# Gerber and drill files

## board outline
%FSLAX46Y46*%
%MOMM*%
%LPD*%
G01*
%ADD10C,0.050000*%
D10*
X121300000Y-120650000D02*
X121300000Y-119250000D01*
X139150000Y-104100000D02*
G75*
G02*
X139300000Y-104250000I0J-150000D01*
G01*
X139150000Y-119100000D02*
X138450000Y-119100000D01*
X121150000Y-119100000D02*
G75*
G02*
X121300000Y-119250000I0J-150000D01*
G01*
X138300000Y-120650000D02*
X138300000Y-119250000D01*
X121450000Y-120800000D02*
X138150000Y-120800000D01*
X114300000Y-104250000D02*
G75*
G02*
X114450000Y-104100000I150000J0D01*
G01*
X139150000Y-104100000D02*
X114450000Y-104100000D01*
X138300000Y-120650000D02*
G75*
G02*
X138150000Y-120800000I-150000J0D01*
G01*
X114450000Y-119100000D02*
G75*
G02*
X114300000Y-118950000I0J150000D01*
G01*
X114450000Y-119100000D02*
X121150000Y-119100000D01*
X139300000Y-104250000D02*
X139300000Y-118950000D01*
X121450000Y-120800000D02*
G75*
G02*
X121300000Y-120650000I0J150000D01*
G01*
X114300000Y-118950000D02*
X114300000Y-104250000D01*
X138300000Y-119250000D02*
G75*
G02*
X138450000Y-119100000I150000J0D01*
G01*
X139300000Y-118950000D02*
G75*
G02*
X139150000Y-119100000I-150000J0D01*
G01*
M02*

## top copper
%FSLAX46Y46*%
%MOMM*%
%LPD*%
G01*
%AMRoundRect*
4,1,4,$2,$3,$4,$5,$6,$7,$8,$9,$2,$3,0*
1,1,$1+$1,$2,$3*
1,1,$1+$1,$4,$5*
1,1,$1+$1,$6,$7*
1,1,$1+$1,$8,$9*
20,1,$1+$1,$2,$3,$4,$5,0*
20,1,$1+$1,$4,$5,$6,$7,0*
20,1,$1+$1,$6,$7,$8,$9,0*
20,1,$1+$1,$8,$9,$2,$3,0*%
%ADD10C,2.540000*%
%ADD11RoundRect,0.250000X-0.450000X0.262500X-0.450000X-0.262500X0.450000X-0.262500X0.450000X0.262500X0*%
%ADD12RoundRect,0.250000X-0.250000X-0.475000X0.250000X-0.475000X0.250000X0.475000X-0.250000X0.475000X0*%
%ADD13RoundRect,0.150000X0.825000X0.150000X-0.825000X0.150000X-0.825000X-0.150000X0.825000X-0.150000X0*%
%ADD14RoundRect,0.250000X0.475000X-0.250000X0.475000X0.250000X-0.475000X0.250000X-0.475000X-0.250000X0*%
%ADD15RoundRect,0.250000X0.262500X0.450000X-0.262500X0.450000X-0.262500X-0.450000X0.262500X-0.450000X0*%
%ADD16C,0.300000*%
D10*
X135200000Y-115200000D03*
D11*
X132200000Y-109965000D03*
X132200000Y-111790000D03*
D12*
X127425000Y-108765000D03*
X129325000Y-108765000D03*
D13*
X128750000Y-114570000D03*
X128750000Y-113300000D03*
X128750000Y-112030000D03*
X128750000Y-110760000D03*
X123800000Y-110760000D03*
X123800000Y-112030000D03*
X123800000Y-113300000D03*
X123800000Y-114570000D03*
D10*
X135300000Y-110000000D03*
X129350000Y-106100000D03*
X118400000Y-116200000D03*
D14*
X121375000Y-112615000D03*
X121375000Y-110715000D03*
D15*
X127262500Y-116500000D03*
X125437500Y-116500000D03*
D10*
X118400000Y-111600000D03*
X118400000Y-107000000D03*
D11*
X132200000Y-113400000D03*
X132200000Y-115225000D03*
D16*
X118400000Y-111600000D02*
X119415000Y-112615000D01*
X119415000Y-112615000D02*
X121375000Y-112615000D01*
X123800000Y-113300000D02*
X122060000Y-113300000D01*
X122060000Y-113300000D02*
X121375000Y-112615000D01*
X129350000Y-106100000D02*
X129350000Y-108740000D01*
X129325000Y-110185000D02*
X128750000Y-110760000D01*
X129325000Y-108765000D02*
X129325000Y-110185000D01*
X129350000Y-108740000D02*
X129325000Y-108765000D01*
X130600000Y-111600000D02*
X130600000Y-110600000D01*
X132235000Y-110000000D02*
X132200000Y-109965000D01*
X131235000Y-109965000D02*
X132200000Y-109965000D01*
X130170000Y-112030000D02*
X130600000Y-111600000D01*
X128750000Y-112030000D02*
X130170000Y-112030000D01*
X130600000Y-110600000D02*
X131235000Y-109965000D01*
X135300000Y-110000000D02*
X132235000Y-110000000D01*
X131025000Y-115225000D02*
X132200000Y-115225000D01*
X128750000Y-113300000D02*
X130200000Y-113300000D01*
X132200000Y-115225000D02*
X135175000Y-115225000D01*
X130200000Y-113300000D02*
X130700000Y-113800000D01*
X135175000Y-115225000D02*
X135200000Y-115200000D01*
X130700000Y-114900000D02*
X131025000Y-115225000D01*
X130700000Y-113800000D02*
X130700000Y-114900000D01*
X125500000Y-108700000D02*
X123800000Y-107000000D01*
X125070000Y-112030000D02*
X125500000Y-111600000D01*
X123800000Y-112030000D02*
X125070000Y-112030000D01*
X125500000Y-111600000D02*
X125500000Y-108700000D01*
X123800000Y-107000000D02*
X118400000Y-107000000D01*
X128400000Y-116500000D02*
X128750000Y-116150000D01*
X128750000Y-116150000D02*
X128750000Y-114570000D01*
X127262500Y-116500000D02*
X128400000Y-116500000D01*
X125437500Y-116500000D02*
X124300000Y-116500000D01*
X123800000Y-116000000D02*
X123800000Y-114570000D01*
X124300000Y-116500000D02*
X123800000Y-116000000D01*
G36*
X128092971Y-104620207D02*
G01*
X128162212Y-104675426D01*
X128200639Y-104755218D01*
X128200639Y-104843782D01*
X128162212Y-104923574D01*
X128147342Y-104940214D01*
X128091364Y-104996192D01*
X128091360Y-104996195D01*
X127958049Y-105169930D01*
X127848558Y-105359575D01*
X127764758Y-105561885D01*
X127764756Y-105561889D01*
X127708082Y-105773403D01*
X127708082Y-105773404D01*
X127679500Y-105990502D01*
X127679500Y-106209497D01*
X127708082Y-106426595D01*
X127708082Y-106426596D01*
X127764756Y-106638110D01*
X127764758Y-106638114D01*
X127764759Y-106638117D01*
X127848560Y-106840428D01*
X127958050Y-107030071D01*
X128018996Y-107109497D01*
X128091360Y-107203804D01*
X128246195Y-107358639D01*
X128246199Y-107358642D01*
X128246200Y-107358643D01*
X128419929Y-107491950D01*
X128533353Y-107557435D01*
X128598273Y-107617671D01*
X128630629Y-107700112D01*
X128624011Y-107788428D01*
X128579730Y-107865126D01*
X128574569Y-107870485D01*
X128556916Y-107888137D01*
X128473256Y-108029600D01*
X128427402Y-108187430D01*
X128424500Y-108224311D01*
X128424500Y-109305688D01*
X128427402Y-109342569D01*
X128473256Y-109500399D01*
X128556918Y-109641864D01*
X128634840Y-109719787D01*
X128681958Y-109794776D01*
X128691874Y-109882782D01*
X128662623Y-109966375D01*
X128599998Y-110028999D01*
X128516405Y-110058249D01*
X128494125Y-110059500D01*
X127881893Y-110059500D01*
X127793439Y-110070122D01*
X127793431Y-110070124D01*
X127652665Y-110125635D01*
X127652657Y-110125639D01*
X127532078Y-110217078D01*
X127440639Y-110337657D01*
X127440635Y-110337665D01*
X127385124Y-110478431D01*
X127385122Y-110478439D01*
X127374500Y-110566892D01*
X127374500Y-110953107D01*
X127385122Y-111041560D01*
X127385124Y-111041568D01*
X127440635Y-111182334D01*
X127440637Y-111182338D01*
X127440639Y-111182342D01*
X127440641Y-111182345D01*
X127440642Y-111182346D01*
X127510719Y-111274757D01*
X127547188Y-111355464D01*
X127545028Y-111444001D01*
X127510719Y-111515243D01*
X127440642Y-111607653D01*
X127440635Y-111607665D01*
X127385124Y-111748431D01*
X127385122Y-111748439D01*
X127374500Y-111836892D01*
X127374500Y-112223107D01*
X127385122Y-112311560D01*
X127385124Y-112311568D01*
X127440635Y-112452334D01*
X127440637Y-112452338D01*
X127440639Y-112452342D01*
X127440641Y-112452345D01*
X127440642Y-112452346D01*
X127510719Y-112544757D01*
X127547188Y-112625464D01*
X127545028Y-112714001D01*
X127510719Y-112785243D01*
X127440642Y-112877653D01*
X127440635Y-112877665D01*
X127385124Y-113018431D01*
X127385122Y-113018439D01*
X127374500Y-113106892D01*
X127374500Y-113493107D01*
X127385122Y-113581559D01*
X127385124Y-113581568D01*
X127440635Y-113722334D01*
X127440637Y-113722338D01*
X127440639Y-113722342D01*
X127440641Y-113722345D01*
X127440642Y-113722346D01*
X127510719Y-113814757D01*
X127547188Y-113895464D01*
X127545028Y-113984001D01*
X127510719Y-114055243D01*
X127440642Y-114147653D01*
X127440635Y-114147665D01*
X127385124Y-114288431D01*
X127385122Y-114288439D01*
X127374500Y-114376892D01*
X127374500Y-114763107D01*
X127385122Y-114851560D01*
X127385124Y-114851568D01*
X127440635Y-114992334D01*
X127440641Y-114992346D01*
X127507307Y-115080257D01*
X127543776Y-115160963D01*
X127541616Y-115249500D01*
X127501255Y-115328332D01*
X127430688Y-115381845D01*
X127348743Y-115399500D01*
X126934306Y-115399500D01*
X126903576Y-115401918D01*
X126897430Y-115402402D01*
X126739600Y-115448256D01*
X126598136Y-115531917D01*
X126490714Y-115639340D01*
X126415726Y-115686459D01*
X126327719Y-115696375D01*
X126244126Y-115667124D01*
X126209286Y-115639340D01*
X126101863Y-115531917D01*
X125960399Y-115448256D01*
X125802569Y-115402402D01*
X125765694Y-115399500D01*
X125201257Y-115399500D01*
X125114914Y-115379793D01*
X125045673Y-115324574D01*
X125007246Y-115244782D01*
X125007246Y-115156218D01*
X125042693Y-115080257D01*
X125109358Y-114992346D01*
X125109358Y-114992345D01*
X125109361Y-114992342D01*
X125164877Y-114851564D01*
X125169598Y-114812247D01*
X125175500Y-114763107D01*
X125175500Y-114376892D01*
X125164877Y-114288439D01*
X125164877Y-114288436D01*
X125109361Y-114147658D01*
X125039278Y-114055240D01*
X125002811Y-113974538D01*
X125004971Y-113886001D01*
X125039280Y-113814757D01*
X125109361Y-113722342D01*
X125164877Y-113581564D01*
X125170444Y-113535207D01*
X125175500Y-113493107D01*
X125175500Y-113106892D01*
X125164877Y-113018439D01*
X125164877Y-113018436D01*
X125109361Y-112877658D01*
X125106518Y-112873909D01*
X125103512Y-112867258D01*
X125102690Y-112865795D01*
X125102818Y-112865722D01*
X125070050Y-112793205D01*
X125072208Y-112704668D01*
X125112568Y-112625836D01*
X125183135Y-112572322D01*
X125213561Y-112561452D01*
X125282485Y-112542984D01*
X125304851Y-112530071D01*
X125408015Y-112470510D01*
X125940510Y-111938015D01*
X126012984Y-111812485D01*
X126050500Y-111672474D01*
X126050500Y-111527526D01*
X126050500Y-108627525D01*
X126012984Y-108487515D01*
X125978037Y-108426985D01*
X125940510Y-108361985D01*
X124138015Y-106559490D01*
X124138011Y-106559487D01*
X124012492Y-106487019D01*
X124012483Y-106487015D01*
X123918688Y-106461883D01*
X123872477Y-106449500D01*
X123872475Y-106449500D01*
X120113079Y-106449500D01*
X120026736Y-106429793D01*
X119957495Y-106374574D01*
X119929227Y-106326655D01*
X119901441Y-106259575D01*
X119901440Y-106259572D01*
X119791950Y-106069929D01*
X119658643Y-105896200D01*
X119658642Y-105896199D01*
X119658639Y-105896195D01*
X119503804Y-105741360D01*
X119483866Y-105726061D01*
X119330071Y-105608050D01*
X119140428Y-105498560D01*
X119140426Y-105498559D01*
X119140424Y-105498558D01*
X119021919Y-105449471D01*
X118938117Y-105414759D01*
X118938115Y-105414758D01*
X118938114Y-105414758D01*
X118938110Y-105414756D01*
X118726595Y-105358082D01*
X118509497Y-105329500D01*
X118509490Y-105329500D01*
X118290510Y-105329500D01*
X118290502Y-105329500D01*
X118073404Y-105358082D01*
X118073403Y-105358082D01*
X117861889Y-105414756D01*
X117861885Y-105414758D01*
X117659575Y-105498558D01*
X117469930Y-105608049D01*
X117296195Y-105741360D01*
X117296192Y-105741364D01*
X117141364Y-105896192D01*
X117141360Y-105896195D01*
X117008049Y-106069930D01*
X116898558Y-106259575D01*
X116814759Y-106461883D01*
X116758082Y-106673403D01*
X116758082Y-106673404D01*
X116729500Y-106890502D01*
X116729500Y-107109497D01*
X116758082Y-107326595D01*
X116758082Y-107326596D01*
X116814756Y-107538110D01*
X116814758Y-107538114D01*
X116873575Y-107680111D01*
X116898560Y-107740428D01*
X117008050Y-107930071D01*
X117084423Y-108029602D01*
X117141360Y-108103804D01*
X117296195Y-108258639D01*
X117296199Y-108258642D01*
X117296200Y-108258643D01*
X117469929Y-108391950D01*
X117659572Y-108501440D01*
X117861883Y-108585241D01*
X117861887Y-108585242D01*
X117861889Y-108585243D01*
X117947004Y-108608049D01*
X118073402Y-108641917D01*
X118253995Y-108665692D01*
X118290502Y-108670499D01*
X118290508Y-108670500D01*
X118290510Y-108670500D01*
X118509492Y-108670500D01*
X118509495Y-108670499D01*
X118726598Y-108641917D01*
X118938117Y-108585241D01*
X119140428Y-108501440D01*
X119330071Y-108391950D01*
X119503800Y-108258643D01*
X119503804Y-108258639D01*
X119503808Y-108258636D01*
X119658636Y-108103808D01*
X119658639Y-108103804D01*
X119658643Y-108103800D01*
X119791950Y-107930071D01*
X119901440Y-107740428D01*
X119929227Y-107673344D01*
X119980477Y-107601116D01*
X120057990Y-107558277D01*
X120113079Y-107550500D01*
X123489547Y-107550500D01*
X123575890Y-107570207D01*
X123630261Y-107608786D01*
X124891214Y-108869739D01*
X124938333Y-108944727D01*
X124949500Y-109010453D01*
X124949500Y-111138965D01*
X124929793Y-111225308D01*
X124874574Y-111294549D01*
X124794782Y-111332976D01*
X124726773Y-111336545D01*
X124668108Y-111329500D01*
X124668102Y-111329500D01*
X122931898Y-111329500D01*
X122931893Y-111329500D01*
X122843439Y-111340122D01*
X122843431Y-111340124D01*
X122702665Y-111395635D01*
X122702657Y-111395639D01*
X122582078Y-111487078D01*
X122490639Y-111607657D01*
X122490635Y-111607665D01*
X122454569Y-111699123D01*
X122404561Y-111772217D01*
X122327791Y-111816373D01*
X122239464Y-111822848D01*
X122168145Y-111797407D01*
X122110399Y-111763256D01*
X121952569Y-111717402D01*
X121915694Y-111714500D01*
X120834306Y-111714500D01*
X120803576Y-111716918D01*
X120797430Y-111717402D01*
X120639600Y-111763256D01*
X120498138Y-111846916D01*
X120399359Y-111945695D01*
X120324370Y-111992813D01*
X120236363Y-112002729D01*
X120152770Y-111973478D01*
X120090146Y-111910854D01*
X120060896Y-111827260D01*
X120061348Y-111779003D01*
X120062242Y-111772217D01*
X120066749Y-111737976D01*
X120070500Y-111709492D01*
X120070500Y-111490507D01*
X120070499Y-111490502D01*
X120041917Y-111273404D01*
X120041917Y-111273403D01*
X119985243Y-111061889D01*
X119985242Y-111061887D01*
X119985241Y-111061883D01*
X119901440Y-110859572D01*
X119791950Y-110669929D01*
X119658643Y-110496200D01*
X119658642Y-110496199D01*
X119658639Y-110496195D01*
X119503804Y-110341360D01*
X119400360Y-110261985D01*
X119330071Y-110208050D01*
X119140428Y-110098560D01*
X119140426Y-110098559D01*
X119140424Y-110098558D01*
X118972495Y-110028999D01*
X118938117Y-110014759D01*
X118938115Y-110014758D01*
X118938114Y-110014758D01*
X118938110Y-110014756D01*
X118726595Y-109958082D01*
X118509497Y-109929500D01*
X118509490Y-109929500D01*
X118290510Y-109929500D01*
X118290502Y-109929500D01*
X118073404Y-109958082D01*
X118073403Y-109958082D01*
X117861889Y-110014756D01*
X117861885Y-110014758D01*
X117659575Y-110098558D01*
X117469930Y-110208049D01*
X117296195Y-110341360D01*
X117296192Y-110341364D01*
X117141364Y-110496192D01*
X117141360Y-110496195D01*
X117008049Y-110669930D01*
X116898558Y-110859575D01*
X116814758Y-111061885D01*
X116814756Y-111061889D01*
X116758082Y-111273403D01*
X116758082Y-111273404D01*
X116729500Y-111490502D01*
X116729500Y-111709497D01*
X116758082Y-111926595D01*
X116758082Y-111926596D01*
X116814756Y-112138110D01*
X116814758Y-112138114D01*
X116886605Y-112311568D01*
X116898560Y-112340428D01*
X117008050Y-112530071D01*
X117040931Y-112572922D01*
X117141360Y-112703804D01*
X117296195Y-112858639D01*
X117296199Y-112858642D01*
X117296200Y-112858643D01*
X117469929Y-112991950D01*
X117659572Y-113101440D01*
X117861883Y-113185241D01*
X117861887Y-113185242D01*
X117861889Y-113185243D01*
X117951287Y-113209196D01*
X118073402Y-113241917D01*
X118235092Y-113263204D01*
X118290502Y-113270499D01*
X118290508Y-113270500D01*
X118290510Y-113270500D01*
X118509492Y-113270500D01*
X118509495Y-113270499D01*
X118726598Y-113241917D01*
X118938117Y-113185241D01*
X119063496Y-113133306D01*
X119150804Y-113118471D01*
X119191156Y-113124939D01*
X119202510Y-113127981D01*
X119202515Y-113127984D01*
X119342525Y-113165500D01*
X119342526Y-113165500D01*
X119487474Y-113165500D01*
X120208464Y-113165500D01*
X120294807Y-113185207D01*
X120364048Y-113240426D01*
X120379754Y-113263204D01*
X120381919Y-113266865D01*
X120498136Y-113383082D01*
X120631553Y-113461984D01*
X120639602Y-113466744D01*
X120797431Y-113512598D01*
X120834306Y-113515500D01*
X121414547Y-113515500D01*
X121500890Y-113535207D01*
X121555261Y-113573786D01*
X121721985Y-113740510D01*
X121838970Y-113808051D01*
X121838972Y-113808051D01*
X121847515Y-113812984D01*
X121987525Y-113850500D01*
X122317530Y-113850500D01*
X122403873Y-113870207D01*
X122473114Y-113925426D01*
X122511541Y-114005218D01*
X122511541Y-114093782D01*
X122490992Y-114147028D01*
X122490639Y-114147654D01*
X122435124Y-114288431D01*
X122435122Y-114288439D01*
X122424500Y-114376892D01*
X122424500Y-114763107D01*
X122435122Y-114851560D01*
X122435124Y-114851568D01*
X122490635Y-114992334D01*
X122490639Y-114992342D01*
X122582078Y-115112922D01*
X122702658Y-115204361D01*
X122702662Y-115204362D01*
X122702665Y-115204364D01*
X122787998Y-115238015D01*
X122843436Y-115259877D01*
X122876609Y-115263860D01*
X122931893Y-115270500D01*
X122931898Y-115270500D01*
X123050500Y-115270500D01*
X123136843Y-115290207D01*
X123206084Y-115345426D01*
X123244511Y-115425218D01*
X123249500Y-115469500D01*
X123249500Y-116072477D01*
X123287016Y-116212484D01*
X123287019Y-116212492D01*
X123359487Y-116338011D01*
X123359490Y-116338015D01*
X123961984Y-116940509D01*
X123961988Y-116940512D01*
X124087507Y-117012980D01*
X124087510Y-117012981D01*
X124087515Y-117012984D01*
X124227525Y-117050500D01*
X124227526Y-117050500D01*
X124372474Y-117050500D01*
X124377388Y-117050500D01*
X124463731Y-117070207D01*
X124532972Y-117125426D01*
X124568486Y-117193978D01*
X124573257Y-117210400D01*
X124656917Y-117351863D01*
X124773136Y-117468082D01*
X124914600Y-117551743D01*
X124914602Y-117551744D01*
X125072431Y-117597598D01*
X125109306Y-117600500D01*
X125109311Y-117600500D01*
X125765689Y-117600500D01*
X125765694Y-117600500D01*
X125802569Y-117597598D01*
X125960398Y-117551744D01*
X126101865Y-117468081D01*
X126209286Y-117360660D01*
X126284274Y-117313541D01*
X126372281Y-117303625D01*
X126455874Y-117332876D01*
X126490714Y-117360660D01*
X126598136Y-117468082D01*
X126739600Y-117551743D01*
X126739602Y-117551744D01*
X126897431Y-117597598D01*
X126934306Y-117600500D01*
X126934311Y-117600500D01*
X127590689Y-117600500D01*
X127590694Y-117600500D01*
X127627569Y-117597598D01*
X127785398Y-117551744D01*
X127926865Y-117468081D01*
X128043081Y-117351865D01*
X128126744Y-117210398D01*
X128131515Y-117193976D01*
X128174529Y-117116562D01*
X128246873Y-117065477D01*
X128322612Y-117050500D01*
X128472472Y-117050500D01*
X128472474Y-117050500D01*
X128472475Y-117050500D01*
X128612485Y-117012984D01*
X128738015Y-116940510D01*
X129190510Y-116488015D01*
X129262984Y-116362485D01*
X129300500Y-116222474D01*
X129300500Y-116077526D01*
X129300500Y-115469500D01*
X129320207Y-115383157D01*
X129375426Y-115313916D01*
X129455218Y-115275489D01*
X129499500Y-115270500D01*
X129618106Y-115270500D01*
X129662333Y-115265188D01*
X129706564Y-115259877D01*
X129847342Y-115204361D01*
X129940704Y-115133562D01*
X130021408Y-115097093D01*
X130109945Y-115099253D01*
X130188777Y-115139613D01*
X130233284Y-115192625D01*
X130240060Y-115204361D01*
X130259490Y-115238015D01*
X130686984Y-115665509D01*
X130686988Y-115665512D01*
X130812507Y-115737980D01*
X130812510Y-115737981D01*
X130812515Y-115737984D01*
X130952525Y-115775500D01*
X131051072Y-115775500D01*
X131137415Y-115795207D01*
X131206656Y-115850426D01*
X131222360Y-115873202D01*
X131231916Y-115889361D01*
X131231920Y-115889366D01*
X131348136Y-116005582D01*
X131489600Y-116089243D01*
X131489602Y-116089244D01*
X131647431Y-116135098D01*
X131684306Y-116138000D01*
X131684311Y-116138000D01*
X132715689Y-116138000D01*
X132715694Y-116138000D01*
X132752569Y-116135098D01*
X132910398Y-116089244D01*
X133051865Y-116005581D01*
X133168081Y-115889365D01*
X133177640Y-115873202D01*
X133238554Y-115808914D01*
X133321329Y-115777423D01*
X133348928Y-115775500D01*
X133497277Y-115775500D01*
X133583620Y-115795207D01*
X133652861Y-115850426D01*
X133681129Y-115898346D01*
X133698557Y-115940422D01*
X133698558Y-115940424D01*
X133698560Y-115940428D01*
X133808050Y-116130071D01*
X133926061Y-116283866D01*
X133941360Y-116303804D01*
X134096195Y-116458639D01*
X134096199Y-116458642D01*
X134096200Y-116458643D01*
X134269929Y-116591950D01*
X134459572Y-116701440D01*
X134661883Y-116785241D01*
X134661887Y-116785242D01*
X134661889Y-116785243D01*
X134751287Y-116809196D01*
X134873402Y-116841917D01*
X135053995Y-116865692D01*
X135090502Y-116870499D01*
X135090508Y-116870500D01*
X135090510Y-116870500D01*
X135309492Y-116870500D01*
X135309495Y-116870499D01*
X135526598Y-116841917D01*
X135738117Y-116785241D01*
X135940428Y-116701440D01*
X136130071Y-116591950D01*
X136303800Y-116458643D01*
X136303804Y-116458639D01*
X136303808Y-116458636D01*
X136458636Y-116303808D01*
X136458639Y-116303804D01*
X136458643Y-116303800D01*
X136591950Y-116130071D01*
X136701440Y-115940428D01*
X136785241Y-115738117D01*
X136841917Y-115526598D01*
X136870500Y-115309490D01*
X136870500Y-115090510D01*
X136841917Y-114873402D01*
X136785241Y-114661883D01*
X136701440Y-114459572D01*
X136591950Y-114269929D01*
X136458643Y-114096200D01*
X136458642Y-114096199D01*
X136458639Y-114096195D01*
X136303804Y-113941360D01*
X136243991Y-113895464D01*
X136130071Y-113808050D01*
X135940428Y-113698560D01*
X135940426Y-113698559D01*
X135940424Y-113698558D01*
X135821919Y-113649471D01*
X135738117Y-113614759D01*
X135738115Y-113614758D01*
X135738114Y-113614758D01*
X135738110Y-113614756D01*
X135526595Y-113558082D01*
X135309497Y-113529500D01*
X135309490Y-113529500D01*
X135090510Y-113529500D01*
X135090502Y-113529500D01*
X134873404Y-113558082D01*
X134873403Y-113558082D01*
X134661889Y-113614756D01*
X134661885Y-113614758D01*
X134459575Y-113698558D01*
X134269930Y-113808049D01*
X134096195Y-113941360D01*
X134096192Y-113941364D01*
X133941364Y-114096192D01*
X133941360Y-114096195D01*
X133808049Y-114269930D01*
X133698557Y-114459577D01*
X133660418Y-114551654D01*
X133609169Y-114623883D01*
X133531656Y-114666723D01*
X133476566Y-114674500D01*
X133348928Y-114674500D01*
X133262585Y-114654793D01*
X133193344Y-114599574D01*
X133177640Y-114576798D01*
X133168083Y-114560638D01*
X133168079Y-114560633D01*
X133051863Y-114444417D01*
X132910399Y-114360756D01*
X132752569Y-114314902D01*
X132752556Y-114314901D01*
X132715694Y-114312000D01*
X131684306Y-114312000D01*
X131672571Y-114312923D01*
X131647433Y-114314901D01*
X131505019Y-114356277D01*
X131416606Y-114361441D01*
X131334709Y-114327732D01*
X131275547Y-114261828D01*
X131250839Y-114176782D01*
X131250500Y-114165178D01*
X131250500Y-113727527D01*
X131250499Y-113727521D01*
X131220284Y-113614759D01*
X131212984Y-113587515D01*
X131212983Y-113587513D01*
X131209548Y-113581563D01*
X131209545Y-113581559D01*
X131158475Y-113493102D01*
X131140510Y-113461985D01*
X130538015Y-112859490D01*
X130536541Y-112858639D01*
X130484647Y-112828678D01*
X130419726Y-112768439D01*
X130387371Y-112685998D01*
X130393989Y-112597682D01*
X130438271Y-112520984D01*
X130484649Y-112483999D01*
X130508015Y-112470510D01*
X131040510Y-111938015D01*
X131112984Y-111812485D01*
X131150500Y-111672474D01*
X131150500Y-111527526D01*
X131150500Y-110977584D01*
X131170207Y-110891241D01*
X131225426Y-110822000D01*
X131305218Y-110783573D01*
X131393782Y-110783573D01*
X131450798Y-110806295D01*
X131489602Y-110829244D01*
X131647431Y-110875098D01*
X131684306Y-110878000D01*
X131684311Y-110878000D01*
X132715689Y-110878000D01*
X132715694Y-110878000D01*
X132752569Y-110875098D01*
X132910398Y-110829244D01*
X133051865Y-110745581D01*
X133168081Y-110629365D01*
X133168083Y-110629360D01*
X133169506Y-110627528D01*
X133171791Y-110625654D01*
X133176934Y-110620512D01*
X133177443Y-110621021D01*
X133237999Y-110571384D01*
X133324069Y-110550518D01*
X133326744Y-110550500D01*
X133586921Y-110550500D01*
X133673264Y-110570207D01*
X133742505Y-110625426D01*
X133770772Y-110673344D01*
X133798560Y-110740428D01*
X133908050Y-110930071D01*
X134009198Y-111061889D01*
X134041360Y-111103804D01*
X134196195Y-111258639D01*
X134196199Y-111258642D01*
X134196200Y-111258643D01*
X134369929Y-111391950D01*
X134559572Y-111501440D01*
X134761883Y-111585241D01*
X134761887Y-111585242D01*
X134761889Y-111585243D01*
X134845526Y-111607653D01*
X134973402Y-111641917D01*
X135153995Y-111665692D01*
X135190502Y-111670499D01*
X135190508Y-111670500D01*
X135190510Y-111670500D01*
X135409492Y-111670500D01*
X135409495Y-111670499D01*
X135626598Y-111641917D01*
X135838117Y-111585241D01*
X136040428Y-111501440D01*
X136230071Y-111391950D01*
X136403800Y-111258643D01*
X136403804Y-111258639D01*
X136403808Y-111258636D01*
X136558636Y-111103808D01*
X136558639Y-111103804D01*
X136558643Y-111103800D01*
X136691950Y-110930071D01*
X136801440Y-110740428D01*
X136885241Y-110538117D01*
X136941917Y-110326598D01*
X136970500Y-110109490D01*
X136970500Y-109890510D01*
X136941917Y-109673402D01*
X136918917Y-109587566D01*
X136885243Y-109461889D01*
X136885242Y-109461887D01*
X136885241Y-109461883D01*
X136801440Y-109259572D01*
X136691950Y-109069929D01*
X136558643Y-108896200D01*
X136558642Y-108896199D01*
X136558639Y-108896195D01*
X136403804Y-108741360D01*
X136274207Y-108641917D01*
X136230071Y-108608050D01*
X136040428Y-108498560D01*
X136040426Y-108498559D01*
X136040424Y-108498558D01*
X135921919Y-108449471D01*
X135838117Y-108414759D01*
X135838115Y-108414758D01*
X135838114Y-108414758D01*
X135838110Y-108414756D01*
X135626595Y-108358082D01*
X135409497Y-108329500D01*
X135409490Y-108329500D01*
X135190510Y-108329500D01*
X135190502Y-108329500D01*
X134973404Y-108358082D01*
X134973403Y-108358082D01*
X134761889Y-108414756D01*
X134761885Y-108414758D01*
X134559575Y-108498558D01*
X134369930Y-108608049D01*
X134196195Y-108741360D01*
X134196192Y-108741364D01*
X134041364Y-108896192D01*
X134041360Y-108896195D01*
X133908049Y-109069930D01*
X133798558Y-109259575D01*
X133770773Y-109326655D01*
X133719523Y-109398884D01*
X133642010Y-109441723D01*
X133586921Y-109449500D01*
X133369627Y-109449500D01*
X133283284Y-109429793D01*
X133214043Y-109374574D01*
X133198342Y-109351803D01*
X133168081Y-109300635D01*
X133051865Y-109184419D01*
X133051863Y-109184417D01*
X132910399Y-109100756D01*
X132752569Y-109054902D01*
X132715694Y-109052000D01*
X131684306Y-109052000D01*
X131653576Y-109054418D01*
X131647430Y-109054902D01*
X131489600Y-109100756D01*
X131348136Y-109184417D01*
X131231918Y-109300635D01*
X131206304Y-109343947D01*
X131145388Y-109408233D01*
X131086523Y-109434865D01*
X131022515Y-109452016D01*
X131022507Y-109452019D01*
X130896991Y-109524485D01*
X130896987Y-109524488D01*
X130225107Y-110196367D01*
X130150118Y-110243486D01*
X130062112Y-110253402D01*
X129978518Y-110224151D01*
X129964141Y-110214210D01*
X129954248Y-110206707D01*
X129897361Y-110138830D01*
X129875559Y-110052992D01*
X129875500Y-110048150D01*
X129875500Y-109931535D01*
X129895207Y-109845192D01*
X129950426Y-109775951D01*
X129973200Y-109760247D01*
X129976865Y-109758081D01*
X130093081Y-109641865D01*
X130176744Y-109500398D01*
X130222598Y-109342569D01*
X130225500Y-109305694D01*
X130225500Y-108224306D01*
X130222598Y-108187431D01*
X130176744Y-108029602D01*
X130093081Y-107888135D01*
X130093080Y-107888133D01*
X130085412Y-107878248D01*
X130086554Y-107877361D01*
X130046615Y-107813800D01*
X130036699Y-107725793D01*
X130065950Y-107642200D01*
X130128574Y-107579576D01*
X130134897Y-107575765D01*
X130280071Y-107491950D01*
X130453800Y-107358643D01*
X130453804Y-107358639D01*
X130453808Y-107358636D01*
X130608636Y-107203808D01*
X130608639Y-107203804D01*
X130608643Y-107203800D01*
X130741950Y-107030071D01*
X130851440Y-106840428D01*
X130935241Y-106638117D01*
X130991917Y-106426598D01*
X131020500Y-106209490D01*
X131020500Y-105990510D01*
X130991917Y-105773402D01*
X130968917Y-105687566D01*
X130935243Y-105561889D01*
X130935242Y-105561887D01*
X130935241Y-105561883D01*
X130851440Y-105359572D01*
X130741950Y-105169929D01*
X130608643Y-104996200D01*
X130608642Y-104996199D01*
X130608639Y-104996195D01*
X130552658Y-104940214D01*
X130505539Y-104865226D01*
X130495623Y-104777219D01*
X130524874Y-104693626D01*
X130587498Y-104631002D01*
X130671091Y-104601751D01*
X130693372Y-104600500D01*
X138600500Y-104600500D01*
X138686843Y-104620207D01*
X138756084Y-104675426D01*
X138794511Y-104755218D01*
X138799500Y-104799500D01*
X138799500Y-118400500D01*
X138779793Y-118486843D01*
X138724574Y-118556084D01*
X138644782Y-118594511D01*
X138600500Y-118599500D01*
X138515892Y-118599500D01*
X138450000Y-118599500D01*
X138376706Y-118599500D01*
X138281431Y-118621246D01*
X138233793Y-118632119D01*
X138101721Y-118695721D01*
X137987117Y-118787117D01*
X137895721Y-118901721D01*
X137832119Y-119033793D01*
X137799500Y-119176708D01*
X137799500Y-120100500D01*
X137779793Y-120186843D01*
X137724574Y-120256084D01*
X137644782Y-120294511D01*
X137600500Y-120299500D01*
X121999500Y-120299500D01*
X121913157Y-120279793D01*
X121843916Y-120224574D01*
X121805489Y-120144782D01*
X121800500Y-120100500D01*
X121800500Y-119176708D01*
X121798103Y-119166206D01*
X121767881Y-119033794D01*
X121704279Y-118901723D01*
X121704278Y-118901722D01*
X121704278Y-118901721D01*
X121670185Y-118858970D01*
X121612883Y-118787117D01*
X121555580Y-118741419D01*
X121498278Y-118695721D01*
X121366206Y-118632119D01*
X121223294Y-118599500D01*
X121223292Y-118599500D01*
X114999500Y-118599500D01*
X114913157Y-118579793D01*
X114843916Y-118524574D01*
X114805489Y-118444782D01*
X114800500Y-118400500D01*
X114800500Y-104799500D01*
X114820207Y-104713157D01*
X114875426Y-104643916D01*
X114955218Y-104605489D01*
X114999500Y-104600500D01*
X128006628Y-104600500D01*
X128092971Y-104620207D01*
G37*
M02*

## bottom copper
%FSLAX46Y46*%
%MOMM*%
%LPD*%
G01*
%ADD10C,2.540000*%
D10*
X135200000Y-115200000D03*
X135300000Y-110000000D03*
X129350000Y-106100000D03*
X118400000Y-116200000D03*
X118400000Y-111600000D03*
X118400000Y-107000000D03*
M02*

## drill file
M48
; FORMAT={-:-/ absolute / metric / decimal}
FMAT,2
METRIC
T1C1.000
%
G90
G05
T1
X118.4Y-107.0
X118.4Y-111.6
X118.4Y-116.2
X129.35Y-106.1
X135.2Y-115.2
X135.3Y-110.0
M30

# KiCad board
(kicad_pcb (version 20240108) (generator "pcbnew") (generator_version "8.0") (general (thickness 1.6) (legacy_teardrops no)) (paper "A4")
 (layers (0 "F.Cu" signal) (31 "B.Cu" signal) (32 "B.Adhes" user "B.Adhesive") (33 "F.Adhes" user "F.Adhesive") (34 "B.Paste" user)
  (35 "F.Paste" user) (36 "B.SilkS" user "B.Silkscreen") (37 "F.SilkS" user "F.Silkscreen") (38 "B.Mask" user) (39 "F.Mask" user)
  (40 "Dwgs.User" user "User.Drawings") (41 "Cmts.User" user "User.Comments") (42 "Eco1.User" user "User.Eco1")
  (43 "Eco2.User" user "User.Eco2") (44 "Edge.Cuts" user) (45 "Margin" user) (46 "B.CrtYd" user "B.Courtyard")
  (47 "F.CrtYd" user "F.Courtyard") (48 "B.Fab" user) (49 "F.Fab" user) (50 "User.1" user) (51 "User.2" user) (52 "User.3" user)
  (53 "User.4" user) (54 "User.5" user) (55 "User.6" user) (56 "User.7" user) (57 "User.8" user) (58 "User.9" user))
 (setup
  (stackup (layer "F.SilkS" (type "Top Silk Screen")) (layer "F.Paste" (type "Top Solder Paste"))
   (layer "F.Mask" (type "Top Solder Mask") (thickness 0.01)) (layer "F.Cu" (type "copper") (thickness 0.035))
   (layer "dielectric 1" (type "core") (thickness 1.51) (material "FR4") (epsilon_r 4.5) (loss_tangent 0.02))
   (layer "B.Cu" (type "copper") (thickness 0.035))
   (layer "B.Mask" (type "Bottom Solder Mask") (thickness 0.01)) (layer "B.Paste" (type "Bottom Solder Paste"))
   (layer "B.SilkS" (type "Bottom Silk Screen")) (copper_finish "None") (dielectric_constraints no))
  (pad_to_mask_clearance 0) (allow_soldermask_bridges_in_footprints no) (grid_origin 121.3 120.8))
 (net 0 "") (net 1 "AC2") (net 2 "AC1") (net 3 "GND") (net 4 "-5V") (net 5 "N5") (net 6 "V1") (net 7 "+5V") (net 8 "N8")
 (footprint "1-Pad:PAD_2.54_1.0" (layer "F.Cu") (at 135.2 115.2)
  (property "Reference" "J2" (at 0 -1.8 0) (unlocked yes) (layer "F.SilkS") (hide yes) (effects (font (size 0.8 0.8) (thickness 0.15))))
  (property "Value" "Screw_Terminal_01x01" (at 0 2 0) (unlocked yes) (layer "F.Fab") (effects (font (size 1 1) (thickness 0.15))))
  (pad "1" thru_hole circle (at 0 0) (size 2.54 2.54) (drill 1) (layers "*.Cu" "*.Mask") (remove_unused_layers no) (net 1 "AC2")))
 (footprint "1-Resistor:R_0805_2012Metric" (layer "F.Cu") (at 132.2 110.8775 -90)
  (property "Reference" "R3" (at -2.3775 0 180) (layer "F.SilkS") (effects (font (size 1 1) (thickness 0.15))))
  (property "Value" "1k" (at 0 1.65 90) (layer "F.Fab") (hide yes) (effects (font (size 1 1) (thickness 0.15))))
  (pad "1" smd roundrect (at -0.9125 0 270) (size 1.025 1.4) (layers "F.Cu" "F.Paste" "F.Mask") (roundrect_rratio 0.243902) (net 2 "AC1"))
  (pad "2" smd roundrect (at 0.9125 0 270) (size 1.025 1.4) (layers "F.Cu" "F.Paste" "F.Mask") (roundrect_rratio 0.243902) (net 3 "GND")))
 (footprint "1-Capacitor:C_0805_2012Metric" (layer "F.Cu") (at 128.375 108.765)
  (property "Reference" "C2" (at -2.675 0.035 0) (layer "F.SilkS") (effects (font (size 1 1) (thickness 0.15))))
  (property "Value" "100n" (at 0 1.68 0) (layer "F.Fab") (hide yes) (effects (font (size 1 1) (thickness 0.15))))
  (pad "1" smd roundrect (at -0.95 0) (size 1 1.45) (layers "F.Cu" "F.Paste" "F.Mask") (roundrect_rratio 0.25) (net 3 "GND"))
  (pad "2" smd roundrect (at 0.95 0) (size 1 1.45) (layers "F.Cu" "F.Paste" "F.Mask") (roundrect_rratio 0.25) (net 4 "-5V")))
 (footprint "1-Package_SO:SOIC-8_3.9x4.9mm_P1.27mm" (layer "F.Cu") (at 126.275 112.665 180)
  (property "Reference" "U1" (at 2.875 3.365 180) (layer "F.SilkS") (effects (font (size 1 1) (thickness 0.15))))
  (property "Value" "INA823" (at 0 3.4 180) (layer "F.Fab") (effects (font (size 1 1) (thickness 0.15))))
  (pad "1" smd roundrect (at -2.475 -1.905 180) (size 1.95 0.6) (layers "F.Cu" "F.Paste" "F.Mask") (roundrect_rratio 0.25) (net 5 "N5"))
  (pad "2" smd roundrect (at -2.475 -0.635 180) (size 1.95 0.6) (layers "F.Cu" "F.Paste" "F.Mask") (roundrect_rratio 0.25) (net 1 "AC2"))
  (pad "3" smd roundrect (at -2.475 0.635 180) (size 1.95 0.6) (layers "F.Cu" "F.Paste" "F.Mask") (roundrect_rratio 0.25) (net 2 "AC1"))
  (pad "4" smd roundrect (at -2.475 1.905 180) (size 1.95 0.6) (layers "F.Cu" "F.Paste" "F.Mask") (roundrect_rratio 0.25) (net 4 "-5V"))
  (pad "5" smd roundrect (at 2.475 1.905 180) (size 1.95 0.6) (layers "F.Cu" "F.Paste" "F.Mask") (roundrect_rratio 0.25) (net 3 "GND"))
  (pad "6" smd roundrect (at 2.475 0.635 180) (size 1.95 0.6) (layers "F.Cu" "F.Paste" "F.Mask") (roundrect_rratio 0.25) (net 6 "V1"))
  (pad "7" smd roundrect (at 2.475 -0.635 180) (size 1.95 0.6) (layers "F.Cu" "F.Paste" "F.Mask") (roundrect_rratio 0.25) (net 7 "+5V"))
  (pad "8" smd roundrect (at 2.475 -1.905 180) (size 1.95 0.6) (layers "F.Cu" "F.Paste" "F.Mask") (roundrect_rratio 0.25) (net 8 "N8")))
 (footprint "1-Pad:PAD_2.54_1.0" (layer "F.Cu") (at 135.3 110)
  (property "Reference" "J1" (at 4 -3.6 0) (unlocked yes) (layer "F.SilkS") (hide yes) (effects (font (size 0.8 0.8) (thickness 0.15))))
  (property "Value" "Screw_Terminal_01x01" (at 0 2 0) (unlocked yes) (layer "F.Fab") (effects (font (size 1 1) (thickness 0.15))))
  (pad "1" thru_hole circle (at 0 0) (size 2.54 2.54) (drill 1) (layers "*.Cu" "*.Mask") (remove_unused_layers no) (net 2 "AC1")))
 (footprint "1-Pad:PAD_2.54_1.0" (layer "F.Cu") (at 129.35 106.1)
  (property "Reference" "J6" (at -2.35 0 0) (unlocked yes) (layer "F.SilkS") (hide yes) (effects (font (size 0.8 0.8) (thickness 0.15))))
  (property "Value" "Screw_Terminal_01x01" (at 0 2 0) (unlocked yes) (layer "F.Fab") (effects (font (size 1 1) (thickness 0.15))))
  (pad "1" thru_hole circle (at 0 0) (size 2.54 2.54) (drill 1) (layers "*.Cu" "*.Mask") (remove_unused_layers no) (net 4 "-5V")))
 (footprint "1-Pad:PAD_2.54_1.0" (layer "F.Cu") (at 118.4 116.2)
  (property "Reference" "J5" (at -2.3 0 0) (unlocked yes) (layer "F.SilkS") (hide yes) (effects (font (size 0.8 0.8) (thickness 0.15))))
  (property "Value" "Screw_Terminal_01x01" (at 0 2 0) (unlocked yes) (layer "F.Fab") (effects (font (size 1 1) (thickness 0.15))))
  (pad "1" thru_hole circle (at 0 0) (size 2.54 2.54) (drill 1) (layers "*.Cu" "*.Mask") (remove_unused_layers no) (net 3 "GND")))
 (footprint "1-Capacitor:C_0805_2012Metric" (layer "F.Cu") (at 121.375 111.665 90)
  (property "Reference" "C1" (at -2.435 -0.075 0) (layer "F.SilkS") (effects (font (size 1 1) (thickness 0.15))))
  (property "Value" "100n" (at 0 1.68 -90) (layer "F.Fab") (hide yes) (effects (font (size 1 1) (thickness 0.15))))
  (pad "1" smd roundrect (at -0.95 0 90) (size 1 1.45) (layers "F.Cu" "F.Paste" "F.Mask") (roundrect_rratio 0.25) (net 7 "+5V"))
  (pad "2" smd roundrect (at 0.95 0 90) (size 1 1.45) (layers "F.Cu" "F.Paste" "F.Mask") (roundrect_rratio 0.25) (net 3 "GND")))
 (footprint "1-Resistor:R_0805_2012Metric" (layer "F.Cu") (at 126.35 116.5 180)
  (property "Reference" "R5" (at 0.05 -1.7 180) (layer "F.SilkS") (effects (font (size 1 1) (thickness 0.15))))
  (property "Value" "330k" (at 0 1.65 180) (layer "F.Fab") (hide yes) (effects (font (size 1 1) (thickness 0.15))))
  (pad "1" smd roundrect (at -0.9125 0 180) (size 1.025 1.4) (layers "F.Cu" "F.Paste" "F.Mask") (roundrect_rratio 0.243902) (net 5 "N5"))
  (pad "2" smd roundrect (at 0.9125 0 180) (size 1.025 1.4) (layers "F.Cu" "F.Paste" "F.Mask") (roundrect_rratio 0.243902) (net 8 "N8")))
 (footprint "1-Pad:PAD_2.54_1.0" (layer "F.Cu") (at 118.4 111.6)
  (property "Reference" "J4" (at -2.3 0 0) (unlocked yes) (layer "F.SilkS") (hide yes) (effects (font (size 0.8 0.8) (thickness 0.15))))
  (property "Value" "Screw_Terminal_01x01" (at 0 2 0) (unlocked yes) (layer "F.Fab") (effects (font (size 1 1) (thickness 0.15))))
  (pad "1" thru_hole circle (at 0 0) (size 2.54 2.54) (drill 1) (layers "*.Cu" "*.Mask") (remove_unused_layers no) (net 7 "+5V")))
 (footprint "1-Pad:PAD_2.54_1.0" (layer "F.Cu") (at 118.4 107)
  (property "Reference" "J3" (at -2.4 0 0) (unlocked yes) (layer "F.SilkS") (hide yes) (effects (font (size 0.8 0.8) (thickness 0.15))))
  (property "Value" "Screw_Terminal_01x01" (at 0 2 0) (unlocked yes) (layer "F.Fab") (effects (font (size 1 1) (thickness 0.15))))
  (pad "1" thru_hole circle (at 0 0) (size 2.54 2.54) (drill 1) (layers "*.Cu" "*.Mask") (remove_unused_layers no) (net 6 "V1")))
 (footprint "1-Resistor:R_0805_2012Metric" (layer "F.Cu") (at 132.2 114.3125 -90)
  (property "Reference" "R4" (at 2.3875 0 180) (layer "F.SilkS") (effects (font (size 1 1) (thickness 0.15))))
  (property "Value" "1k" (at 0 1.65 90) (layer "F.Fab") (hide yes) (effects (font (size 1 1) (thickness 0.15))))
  (pad "1" smd roundrect (at -0.9125 0 270) (size 1.025 1.4) (layers "F.Cu" "F.Paste" "F.Mask") (roundrect_rratio 0.243902) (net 3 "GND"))
  (pad "2" smd roundrect (at 0.9125 0 270) (size 1.025 1.4) (layers "F.Cu" "F.Paste" "F.Mask") (roundrect_rratio 0.243902) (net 1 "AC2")))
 (gr_line (start 121.3 120.65) (end 121.3 119.25) (stroke (width 0.05) (type default)) (layer "Edge.Cuts"))
 (gr_arc (start 139.15 104.1) (mid 139.256066 104.143934) (end 139.3 104.25) (stroke (width 0.05) (type default)) (layer "Edge.Cuts"))
 (gr_line (start 139.15 119.1) (end 138.45 119.1) (stroke (width 0.05) (type default)) (layer "Edge.Cuts"))
 (gr_arc (start 121.15 119.1) (mid 121.256066 119.143934) (end 121.3 119.25) (stroke (width 0.05) (type default)) (layer "Edge.Cuts"))
 (gr_line (start 138.3 120.65) (end 138.3 119.25) (stroke (width 0.05) (type default)) (layer "Edge.Cuts"))
 (gr_line (start 121.45 120.8) (end 138.15 120.8) (stroke (width 0.05) (type default)) (layer "Edge.Cuts"))
 (gr_arc (start 114.3 104.25) (mid 114.343934 104.143934) (end 114.45 104.1) (stroke (width 0.05) (type default)) (layer "Edge.Cuts"))
 (gr_line (start 139.15 104.1) (end 114.45 104.1) (stroke (width 0.05) (type default)) (layer "Edge.Cuts"))
 (gr_arc (start 138.3 120.65) (mid 138.256066 120.756066) (end 138.15 120.8) (stroke (width 0.05) (type default)) (layer "Edge.Cuts"))
 (gr_arc (start 114.45 119.1) (mid 114.343934 119.056066) (end 114.3 118.95) (stroke (width 0.05) (type default)) (layer "Edge.Cuts"))
 (gr_line (start 114.45 119.1) (end 121.15 119.1) (stroke (width 0.05) (type default)) (layer "Edge.Cuts"))
 (gr_line (start 139.3 104.25) (end 139.3 118.95) (stroke (width 0.05) (type default)) (layer "Edge.Cuts"))
 (gr_arc (start 121.45 120.8) (mid 121.343934 120.756066) (end 121.3 120.65) (stroke (width 0.05) (type default)) (layer "Edge.Cuts"))
 (gr_line (start 114.3 118.95) (end 114.3 104.25) (stroke (width 0.05) (type default)) (layer "Edge.Cuts"))
 (gr_arc (start 138.3 119.25) (mid 138.343934 119.143934) (end 138.45 119.1) (stroke (width 0.05) (type default)) (layer "Edge.Cuts"))
 (gr_arc (start 139.3 118.95) (mid 139.256066 119.056066) (end 139.15 119.1) (stroke (width 0.05) (type default)) (layer "Edge.Cuts"))
 (segment (start 118.4 111.6) (end 119.415 112.615) (width 0.3) (layer "F.Cu") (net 7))
 (segment (start 119.415 112.615) (end 121.375 112.615) (width 0.3) (layer "F.Cu") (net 7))
 (segment (start 123.8 113.3) (end 122.06 113.3) (width 0.3) (layer "F.Cu") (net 7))
 (segment (start 122.06 113.3) (end 121.375 112.615) (width 0.3) (layer "F.Cu") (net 7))
 (segment (start 129.35 106.1) (end 129.35 108.74) (width 0.3) (layer "F.Cu") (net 4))
 (segment (start 129.325 110.185) (end 128.75 110.76) (width 0.3) (layer "F.Cu") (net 4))
 (segment (start 129.325 108.765) (end 129.325 110.185) (width 0.3) (layer "F.Cu") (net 4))
 (segment (start 129.35 108.74) (end 129.325 108.765) (width 0.3) (layer "F.Cu") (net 4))
 (segment (start 130.6 111.6) (end 130.6 110.6) (width 0.3) (layer "F.Cu") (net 2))
 (segment (start 132.235 110) (end 132.2 109.965) (width 0.3) (layer "F.Cu") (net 2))
 (segment (start 131.235 109.965) (end 132.2 109.965) (width 0.3) (layer "F.Cu") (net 2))
 (segment (start 130.17 112.03) (end 130.6 111.6) (width 0.3) (layer "F.Cu") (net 2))
 (segment (start 128.75 112.03) (end 130.17 112.03) (width 0.3) (layer "F.Cu") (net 2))
 (segment (start 130.6 110.6) (end 131.235 109.965) (width 0.3) (layer "F.Cu") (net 2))
 (segment (start 135.3 110) (end 132.235 110) (width 0.3) (layer "F.Cu") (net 2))
 (segment (start 131.025 115.225) (end 132.2 115.225) (width 0.3) (layer "F.Cu") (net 1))
 (segment (start 128.75 113.3) (end 130.2 113.3) (width 0.3) (layer "F.Cu") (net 1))
 (segment (start 132.2 115.225) (end 135.175 115.225) (width 0.3) (layer "F.Cu") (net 1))
 (segment (start 130.2 113.3) (end 130.7 113.8) (width 0.3) (layer "F.Cu") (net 1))
 (segment (start 135.175 115.225) (end 135.2 115.2) (width 0.3) (layer "F.Cu") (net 1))
 (segment (start 130.7 114.9) (end 131.025 115.225) (width 0.3) (layer "F.Cu") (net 1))
 (segment (start 130.7 113.8) (end 130.7 114.9) (width 0.3) (layer "F.Cu") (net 1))
 (segment (start 125.5 108.7) (end 123.8 107) (width 0.3) (layer "F.Cu") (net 6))
 (segment (start 125.07 112.03) (end 125.5 111.6) (width 0.3) (layer "F.Cu") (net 6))
 (segment (start 123.8 112.03) (end 125.07 112.03) (width 0.3) (layer "F.Cu") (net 6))
 (segment (start 125.5 111.6) (end 125.5 108.7) (width 0.3) (layer "F.Cu") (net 6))
 (segment (start 123.8 107) (end 118.4 107) (width 0.3) (layer "F.Cu") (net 6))
 (segment (start 128.4 116.5) (end 128.75 116.15) (width 0.3) (layer "F.Cu") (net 5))
 (segment (start 128.75 116.15) (end 128.75 114.57) (width 0.3) (layer "F.Cu") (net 5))
 (segment (start 127.2625 116.5) (end 128.4 116.5) (width 0.3) (layer "F.Cu") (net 5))
 (segment (start 125.4375 116.5) (end 124.3 116.5) (width 0.3) (layer "F.Cu") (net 8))
 (segment (start 123.8 116) (end 123.8 114.57) (width 0.3) (layer "F.Cu") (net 8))
 (segment (start 124.3 116.5) (end 123.8 116) (width 0.3) (layer "F.Cu") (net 8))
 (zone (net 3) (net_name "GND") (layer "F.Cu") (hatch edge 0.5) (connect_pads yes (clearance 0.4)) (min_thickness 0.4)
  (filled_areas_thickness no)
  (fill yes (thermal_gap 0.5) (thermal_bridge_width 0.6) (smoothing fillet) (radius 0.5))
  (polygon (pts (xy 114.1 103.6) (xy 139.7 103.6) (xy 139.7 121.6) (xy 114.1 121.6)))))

